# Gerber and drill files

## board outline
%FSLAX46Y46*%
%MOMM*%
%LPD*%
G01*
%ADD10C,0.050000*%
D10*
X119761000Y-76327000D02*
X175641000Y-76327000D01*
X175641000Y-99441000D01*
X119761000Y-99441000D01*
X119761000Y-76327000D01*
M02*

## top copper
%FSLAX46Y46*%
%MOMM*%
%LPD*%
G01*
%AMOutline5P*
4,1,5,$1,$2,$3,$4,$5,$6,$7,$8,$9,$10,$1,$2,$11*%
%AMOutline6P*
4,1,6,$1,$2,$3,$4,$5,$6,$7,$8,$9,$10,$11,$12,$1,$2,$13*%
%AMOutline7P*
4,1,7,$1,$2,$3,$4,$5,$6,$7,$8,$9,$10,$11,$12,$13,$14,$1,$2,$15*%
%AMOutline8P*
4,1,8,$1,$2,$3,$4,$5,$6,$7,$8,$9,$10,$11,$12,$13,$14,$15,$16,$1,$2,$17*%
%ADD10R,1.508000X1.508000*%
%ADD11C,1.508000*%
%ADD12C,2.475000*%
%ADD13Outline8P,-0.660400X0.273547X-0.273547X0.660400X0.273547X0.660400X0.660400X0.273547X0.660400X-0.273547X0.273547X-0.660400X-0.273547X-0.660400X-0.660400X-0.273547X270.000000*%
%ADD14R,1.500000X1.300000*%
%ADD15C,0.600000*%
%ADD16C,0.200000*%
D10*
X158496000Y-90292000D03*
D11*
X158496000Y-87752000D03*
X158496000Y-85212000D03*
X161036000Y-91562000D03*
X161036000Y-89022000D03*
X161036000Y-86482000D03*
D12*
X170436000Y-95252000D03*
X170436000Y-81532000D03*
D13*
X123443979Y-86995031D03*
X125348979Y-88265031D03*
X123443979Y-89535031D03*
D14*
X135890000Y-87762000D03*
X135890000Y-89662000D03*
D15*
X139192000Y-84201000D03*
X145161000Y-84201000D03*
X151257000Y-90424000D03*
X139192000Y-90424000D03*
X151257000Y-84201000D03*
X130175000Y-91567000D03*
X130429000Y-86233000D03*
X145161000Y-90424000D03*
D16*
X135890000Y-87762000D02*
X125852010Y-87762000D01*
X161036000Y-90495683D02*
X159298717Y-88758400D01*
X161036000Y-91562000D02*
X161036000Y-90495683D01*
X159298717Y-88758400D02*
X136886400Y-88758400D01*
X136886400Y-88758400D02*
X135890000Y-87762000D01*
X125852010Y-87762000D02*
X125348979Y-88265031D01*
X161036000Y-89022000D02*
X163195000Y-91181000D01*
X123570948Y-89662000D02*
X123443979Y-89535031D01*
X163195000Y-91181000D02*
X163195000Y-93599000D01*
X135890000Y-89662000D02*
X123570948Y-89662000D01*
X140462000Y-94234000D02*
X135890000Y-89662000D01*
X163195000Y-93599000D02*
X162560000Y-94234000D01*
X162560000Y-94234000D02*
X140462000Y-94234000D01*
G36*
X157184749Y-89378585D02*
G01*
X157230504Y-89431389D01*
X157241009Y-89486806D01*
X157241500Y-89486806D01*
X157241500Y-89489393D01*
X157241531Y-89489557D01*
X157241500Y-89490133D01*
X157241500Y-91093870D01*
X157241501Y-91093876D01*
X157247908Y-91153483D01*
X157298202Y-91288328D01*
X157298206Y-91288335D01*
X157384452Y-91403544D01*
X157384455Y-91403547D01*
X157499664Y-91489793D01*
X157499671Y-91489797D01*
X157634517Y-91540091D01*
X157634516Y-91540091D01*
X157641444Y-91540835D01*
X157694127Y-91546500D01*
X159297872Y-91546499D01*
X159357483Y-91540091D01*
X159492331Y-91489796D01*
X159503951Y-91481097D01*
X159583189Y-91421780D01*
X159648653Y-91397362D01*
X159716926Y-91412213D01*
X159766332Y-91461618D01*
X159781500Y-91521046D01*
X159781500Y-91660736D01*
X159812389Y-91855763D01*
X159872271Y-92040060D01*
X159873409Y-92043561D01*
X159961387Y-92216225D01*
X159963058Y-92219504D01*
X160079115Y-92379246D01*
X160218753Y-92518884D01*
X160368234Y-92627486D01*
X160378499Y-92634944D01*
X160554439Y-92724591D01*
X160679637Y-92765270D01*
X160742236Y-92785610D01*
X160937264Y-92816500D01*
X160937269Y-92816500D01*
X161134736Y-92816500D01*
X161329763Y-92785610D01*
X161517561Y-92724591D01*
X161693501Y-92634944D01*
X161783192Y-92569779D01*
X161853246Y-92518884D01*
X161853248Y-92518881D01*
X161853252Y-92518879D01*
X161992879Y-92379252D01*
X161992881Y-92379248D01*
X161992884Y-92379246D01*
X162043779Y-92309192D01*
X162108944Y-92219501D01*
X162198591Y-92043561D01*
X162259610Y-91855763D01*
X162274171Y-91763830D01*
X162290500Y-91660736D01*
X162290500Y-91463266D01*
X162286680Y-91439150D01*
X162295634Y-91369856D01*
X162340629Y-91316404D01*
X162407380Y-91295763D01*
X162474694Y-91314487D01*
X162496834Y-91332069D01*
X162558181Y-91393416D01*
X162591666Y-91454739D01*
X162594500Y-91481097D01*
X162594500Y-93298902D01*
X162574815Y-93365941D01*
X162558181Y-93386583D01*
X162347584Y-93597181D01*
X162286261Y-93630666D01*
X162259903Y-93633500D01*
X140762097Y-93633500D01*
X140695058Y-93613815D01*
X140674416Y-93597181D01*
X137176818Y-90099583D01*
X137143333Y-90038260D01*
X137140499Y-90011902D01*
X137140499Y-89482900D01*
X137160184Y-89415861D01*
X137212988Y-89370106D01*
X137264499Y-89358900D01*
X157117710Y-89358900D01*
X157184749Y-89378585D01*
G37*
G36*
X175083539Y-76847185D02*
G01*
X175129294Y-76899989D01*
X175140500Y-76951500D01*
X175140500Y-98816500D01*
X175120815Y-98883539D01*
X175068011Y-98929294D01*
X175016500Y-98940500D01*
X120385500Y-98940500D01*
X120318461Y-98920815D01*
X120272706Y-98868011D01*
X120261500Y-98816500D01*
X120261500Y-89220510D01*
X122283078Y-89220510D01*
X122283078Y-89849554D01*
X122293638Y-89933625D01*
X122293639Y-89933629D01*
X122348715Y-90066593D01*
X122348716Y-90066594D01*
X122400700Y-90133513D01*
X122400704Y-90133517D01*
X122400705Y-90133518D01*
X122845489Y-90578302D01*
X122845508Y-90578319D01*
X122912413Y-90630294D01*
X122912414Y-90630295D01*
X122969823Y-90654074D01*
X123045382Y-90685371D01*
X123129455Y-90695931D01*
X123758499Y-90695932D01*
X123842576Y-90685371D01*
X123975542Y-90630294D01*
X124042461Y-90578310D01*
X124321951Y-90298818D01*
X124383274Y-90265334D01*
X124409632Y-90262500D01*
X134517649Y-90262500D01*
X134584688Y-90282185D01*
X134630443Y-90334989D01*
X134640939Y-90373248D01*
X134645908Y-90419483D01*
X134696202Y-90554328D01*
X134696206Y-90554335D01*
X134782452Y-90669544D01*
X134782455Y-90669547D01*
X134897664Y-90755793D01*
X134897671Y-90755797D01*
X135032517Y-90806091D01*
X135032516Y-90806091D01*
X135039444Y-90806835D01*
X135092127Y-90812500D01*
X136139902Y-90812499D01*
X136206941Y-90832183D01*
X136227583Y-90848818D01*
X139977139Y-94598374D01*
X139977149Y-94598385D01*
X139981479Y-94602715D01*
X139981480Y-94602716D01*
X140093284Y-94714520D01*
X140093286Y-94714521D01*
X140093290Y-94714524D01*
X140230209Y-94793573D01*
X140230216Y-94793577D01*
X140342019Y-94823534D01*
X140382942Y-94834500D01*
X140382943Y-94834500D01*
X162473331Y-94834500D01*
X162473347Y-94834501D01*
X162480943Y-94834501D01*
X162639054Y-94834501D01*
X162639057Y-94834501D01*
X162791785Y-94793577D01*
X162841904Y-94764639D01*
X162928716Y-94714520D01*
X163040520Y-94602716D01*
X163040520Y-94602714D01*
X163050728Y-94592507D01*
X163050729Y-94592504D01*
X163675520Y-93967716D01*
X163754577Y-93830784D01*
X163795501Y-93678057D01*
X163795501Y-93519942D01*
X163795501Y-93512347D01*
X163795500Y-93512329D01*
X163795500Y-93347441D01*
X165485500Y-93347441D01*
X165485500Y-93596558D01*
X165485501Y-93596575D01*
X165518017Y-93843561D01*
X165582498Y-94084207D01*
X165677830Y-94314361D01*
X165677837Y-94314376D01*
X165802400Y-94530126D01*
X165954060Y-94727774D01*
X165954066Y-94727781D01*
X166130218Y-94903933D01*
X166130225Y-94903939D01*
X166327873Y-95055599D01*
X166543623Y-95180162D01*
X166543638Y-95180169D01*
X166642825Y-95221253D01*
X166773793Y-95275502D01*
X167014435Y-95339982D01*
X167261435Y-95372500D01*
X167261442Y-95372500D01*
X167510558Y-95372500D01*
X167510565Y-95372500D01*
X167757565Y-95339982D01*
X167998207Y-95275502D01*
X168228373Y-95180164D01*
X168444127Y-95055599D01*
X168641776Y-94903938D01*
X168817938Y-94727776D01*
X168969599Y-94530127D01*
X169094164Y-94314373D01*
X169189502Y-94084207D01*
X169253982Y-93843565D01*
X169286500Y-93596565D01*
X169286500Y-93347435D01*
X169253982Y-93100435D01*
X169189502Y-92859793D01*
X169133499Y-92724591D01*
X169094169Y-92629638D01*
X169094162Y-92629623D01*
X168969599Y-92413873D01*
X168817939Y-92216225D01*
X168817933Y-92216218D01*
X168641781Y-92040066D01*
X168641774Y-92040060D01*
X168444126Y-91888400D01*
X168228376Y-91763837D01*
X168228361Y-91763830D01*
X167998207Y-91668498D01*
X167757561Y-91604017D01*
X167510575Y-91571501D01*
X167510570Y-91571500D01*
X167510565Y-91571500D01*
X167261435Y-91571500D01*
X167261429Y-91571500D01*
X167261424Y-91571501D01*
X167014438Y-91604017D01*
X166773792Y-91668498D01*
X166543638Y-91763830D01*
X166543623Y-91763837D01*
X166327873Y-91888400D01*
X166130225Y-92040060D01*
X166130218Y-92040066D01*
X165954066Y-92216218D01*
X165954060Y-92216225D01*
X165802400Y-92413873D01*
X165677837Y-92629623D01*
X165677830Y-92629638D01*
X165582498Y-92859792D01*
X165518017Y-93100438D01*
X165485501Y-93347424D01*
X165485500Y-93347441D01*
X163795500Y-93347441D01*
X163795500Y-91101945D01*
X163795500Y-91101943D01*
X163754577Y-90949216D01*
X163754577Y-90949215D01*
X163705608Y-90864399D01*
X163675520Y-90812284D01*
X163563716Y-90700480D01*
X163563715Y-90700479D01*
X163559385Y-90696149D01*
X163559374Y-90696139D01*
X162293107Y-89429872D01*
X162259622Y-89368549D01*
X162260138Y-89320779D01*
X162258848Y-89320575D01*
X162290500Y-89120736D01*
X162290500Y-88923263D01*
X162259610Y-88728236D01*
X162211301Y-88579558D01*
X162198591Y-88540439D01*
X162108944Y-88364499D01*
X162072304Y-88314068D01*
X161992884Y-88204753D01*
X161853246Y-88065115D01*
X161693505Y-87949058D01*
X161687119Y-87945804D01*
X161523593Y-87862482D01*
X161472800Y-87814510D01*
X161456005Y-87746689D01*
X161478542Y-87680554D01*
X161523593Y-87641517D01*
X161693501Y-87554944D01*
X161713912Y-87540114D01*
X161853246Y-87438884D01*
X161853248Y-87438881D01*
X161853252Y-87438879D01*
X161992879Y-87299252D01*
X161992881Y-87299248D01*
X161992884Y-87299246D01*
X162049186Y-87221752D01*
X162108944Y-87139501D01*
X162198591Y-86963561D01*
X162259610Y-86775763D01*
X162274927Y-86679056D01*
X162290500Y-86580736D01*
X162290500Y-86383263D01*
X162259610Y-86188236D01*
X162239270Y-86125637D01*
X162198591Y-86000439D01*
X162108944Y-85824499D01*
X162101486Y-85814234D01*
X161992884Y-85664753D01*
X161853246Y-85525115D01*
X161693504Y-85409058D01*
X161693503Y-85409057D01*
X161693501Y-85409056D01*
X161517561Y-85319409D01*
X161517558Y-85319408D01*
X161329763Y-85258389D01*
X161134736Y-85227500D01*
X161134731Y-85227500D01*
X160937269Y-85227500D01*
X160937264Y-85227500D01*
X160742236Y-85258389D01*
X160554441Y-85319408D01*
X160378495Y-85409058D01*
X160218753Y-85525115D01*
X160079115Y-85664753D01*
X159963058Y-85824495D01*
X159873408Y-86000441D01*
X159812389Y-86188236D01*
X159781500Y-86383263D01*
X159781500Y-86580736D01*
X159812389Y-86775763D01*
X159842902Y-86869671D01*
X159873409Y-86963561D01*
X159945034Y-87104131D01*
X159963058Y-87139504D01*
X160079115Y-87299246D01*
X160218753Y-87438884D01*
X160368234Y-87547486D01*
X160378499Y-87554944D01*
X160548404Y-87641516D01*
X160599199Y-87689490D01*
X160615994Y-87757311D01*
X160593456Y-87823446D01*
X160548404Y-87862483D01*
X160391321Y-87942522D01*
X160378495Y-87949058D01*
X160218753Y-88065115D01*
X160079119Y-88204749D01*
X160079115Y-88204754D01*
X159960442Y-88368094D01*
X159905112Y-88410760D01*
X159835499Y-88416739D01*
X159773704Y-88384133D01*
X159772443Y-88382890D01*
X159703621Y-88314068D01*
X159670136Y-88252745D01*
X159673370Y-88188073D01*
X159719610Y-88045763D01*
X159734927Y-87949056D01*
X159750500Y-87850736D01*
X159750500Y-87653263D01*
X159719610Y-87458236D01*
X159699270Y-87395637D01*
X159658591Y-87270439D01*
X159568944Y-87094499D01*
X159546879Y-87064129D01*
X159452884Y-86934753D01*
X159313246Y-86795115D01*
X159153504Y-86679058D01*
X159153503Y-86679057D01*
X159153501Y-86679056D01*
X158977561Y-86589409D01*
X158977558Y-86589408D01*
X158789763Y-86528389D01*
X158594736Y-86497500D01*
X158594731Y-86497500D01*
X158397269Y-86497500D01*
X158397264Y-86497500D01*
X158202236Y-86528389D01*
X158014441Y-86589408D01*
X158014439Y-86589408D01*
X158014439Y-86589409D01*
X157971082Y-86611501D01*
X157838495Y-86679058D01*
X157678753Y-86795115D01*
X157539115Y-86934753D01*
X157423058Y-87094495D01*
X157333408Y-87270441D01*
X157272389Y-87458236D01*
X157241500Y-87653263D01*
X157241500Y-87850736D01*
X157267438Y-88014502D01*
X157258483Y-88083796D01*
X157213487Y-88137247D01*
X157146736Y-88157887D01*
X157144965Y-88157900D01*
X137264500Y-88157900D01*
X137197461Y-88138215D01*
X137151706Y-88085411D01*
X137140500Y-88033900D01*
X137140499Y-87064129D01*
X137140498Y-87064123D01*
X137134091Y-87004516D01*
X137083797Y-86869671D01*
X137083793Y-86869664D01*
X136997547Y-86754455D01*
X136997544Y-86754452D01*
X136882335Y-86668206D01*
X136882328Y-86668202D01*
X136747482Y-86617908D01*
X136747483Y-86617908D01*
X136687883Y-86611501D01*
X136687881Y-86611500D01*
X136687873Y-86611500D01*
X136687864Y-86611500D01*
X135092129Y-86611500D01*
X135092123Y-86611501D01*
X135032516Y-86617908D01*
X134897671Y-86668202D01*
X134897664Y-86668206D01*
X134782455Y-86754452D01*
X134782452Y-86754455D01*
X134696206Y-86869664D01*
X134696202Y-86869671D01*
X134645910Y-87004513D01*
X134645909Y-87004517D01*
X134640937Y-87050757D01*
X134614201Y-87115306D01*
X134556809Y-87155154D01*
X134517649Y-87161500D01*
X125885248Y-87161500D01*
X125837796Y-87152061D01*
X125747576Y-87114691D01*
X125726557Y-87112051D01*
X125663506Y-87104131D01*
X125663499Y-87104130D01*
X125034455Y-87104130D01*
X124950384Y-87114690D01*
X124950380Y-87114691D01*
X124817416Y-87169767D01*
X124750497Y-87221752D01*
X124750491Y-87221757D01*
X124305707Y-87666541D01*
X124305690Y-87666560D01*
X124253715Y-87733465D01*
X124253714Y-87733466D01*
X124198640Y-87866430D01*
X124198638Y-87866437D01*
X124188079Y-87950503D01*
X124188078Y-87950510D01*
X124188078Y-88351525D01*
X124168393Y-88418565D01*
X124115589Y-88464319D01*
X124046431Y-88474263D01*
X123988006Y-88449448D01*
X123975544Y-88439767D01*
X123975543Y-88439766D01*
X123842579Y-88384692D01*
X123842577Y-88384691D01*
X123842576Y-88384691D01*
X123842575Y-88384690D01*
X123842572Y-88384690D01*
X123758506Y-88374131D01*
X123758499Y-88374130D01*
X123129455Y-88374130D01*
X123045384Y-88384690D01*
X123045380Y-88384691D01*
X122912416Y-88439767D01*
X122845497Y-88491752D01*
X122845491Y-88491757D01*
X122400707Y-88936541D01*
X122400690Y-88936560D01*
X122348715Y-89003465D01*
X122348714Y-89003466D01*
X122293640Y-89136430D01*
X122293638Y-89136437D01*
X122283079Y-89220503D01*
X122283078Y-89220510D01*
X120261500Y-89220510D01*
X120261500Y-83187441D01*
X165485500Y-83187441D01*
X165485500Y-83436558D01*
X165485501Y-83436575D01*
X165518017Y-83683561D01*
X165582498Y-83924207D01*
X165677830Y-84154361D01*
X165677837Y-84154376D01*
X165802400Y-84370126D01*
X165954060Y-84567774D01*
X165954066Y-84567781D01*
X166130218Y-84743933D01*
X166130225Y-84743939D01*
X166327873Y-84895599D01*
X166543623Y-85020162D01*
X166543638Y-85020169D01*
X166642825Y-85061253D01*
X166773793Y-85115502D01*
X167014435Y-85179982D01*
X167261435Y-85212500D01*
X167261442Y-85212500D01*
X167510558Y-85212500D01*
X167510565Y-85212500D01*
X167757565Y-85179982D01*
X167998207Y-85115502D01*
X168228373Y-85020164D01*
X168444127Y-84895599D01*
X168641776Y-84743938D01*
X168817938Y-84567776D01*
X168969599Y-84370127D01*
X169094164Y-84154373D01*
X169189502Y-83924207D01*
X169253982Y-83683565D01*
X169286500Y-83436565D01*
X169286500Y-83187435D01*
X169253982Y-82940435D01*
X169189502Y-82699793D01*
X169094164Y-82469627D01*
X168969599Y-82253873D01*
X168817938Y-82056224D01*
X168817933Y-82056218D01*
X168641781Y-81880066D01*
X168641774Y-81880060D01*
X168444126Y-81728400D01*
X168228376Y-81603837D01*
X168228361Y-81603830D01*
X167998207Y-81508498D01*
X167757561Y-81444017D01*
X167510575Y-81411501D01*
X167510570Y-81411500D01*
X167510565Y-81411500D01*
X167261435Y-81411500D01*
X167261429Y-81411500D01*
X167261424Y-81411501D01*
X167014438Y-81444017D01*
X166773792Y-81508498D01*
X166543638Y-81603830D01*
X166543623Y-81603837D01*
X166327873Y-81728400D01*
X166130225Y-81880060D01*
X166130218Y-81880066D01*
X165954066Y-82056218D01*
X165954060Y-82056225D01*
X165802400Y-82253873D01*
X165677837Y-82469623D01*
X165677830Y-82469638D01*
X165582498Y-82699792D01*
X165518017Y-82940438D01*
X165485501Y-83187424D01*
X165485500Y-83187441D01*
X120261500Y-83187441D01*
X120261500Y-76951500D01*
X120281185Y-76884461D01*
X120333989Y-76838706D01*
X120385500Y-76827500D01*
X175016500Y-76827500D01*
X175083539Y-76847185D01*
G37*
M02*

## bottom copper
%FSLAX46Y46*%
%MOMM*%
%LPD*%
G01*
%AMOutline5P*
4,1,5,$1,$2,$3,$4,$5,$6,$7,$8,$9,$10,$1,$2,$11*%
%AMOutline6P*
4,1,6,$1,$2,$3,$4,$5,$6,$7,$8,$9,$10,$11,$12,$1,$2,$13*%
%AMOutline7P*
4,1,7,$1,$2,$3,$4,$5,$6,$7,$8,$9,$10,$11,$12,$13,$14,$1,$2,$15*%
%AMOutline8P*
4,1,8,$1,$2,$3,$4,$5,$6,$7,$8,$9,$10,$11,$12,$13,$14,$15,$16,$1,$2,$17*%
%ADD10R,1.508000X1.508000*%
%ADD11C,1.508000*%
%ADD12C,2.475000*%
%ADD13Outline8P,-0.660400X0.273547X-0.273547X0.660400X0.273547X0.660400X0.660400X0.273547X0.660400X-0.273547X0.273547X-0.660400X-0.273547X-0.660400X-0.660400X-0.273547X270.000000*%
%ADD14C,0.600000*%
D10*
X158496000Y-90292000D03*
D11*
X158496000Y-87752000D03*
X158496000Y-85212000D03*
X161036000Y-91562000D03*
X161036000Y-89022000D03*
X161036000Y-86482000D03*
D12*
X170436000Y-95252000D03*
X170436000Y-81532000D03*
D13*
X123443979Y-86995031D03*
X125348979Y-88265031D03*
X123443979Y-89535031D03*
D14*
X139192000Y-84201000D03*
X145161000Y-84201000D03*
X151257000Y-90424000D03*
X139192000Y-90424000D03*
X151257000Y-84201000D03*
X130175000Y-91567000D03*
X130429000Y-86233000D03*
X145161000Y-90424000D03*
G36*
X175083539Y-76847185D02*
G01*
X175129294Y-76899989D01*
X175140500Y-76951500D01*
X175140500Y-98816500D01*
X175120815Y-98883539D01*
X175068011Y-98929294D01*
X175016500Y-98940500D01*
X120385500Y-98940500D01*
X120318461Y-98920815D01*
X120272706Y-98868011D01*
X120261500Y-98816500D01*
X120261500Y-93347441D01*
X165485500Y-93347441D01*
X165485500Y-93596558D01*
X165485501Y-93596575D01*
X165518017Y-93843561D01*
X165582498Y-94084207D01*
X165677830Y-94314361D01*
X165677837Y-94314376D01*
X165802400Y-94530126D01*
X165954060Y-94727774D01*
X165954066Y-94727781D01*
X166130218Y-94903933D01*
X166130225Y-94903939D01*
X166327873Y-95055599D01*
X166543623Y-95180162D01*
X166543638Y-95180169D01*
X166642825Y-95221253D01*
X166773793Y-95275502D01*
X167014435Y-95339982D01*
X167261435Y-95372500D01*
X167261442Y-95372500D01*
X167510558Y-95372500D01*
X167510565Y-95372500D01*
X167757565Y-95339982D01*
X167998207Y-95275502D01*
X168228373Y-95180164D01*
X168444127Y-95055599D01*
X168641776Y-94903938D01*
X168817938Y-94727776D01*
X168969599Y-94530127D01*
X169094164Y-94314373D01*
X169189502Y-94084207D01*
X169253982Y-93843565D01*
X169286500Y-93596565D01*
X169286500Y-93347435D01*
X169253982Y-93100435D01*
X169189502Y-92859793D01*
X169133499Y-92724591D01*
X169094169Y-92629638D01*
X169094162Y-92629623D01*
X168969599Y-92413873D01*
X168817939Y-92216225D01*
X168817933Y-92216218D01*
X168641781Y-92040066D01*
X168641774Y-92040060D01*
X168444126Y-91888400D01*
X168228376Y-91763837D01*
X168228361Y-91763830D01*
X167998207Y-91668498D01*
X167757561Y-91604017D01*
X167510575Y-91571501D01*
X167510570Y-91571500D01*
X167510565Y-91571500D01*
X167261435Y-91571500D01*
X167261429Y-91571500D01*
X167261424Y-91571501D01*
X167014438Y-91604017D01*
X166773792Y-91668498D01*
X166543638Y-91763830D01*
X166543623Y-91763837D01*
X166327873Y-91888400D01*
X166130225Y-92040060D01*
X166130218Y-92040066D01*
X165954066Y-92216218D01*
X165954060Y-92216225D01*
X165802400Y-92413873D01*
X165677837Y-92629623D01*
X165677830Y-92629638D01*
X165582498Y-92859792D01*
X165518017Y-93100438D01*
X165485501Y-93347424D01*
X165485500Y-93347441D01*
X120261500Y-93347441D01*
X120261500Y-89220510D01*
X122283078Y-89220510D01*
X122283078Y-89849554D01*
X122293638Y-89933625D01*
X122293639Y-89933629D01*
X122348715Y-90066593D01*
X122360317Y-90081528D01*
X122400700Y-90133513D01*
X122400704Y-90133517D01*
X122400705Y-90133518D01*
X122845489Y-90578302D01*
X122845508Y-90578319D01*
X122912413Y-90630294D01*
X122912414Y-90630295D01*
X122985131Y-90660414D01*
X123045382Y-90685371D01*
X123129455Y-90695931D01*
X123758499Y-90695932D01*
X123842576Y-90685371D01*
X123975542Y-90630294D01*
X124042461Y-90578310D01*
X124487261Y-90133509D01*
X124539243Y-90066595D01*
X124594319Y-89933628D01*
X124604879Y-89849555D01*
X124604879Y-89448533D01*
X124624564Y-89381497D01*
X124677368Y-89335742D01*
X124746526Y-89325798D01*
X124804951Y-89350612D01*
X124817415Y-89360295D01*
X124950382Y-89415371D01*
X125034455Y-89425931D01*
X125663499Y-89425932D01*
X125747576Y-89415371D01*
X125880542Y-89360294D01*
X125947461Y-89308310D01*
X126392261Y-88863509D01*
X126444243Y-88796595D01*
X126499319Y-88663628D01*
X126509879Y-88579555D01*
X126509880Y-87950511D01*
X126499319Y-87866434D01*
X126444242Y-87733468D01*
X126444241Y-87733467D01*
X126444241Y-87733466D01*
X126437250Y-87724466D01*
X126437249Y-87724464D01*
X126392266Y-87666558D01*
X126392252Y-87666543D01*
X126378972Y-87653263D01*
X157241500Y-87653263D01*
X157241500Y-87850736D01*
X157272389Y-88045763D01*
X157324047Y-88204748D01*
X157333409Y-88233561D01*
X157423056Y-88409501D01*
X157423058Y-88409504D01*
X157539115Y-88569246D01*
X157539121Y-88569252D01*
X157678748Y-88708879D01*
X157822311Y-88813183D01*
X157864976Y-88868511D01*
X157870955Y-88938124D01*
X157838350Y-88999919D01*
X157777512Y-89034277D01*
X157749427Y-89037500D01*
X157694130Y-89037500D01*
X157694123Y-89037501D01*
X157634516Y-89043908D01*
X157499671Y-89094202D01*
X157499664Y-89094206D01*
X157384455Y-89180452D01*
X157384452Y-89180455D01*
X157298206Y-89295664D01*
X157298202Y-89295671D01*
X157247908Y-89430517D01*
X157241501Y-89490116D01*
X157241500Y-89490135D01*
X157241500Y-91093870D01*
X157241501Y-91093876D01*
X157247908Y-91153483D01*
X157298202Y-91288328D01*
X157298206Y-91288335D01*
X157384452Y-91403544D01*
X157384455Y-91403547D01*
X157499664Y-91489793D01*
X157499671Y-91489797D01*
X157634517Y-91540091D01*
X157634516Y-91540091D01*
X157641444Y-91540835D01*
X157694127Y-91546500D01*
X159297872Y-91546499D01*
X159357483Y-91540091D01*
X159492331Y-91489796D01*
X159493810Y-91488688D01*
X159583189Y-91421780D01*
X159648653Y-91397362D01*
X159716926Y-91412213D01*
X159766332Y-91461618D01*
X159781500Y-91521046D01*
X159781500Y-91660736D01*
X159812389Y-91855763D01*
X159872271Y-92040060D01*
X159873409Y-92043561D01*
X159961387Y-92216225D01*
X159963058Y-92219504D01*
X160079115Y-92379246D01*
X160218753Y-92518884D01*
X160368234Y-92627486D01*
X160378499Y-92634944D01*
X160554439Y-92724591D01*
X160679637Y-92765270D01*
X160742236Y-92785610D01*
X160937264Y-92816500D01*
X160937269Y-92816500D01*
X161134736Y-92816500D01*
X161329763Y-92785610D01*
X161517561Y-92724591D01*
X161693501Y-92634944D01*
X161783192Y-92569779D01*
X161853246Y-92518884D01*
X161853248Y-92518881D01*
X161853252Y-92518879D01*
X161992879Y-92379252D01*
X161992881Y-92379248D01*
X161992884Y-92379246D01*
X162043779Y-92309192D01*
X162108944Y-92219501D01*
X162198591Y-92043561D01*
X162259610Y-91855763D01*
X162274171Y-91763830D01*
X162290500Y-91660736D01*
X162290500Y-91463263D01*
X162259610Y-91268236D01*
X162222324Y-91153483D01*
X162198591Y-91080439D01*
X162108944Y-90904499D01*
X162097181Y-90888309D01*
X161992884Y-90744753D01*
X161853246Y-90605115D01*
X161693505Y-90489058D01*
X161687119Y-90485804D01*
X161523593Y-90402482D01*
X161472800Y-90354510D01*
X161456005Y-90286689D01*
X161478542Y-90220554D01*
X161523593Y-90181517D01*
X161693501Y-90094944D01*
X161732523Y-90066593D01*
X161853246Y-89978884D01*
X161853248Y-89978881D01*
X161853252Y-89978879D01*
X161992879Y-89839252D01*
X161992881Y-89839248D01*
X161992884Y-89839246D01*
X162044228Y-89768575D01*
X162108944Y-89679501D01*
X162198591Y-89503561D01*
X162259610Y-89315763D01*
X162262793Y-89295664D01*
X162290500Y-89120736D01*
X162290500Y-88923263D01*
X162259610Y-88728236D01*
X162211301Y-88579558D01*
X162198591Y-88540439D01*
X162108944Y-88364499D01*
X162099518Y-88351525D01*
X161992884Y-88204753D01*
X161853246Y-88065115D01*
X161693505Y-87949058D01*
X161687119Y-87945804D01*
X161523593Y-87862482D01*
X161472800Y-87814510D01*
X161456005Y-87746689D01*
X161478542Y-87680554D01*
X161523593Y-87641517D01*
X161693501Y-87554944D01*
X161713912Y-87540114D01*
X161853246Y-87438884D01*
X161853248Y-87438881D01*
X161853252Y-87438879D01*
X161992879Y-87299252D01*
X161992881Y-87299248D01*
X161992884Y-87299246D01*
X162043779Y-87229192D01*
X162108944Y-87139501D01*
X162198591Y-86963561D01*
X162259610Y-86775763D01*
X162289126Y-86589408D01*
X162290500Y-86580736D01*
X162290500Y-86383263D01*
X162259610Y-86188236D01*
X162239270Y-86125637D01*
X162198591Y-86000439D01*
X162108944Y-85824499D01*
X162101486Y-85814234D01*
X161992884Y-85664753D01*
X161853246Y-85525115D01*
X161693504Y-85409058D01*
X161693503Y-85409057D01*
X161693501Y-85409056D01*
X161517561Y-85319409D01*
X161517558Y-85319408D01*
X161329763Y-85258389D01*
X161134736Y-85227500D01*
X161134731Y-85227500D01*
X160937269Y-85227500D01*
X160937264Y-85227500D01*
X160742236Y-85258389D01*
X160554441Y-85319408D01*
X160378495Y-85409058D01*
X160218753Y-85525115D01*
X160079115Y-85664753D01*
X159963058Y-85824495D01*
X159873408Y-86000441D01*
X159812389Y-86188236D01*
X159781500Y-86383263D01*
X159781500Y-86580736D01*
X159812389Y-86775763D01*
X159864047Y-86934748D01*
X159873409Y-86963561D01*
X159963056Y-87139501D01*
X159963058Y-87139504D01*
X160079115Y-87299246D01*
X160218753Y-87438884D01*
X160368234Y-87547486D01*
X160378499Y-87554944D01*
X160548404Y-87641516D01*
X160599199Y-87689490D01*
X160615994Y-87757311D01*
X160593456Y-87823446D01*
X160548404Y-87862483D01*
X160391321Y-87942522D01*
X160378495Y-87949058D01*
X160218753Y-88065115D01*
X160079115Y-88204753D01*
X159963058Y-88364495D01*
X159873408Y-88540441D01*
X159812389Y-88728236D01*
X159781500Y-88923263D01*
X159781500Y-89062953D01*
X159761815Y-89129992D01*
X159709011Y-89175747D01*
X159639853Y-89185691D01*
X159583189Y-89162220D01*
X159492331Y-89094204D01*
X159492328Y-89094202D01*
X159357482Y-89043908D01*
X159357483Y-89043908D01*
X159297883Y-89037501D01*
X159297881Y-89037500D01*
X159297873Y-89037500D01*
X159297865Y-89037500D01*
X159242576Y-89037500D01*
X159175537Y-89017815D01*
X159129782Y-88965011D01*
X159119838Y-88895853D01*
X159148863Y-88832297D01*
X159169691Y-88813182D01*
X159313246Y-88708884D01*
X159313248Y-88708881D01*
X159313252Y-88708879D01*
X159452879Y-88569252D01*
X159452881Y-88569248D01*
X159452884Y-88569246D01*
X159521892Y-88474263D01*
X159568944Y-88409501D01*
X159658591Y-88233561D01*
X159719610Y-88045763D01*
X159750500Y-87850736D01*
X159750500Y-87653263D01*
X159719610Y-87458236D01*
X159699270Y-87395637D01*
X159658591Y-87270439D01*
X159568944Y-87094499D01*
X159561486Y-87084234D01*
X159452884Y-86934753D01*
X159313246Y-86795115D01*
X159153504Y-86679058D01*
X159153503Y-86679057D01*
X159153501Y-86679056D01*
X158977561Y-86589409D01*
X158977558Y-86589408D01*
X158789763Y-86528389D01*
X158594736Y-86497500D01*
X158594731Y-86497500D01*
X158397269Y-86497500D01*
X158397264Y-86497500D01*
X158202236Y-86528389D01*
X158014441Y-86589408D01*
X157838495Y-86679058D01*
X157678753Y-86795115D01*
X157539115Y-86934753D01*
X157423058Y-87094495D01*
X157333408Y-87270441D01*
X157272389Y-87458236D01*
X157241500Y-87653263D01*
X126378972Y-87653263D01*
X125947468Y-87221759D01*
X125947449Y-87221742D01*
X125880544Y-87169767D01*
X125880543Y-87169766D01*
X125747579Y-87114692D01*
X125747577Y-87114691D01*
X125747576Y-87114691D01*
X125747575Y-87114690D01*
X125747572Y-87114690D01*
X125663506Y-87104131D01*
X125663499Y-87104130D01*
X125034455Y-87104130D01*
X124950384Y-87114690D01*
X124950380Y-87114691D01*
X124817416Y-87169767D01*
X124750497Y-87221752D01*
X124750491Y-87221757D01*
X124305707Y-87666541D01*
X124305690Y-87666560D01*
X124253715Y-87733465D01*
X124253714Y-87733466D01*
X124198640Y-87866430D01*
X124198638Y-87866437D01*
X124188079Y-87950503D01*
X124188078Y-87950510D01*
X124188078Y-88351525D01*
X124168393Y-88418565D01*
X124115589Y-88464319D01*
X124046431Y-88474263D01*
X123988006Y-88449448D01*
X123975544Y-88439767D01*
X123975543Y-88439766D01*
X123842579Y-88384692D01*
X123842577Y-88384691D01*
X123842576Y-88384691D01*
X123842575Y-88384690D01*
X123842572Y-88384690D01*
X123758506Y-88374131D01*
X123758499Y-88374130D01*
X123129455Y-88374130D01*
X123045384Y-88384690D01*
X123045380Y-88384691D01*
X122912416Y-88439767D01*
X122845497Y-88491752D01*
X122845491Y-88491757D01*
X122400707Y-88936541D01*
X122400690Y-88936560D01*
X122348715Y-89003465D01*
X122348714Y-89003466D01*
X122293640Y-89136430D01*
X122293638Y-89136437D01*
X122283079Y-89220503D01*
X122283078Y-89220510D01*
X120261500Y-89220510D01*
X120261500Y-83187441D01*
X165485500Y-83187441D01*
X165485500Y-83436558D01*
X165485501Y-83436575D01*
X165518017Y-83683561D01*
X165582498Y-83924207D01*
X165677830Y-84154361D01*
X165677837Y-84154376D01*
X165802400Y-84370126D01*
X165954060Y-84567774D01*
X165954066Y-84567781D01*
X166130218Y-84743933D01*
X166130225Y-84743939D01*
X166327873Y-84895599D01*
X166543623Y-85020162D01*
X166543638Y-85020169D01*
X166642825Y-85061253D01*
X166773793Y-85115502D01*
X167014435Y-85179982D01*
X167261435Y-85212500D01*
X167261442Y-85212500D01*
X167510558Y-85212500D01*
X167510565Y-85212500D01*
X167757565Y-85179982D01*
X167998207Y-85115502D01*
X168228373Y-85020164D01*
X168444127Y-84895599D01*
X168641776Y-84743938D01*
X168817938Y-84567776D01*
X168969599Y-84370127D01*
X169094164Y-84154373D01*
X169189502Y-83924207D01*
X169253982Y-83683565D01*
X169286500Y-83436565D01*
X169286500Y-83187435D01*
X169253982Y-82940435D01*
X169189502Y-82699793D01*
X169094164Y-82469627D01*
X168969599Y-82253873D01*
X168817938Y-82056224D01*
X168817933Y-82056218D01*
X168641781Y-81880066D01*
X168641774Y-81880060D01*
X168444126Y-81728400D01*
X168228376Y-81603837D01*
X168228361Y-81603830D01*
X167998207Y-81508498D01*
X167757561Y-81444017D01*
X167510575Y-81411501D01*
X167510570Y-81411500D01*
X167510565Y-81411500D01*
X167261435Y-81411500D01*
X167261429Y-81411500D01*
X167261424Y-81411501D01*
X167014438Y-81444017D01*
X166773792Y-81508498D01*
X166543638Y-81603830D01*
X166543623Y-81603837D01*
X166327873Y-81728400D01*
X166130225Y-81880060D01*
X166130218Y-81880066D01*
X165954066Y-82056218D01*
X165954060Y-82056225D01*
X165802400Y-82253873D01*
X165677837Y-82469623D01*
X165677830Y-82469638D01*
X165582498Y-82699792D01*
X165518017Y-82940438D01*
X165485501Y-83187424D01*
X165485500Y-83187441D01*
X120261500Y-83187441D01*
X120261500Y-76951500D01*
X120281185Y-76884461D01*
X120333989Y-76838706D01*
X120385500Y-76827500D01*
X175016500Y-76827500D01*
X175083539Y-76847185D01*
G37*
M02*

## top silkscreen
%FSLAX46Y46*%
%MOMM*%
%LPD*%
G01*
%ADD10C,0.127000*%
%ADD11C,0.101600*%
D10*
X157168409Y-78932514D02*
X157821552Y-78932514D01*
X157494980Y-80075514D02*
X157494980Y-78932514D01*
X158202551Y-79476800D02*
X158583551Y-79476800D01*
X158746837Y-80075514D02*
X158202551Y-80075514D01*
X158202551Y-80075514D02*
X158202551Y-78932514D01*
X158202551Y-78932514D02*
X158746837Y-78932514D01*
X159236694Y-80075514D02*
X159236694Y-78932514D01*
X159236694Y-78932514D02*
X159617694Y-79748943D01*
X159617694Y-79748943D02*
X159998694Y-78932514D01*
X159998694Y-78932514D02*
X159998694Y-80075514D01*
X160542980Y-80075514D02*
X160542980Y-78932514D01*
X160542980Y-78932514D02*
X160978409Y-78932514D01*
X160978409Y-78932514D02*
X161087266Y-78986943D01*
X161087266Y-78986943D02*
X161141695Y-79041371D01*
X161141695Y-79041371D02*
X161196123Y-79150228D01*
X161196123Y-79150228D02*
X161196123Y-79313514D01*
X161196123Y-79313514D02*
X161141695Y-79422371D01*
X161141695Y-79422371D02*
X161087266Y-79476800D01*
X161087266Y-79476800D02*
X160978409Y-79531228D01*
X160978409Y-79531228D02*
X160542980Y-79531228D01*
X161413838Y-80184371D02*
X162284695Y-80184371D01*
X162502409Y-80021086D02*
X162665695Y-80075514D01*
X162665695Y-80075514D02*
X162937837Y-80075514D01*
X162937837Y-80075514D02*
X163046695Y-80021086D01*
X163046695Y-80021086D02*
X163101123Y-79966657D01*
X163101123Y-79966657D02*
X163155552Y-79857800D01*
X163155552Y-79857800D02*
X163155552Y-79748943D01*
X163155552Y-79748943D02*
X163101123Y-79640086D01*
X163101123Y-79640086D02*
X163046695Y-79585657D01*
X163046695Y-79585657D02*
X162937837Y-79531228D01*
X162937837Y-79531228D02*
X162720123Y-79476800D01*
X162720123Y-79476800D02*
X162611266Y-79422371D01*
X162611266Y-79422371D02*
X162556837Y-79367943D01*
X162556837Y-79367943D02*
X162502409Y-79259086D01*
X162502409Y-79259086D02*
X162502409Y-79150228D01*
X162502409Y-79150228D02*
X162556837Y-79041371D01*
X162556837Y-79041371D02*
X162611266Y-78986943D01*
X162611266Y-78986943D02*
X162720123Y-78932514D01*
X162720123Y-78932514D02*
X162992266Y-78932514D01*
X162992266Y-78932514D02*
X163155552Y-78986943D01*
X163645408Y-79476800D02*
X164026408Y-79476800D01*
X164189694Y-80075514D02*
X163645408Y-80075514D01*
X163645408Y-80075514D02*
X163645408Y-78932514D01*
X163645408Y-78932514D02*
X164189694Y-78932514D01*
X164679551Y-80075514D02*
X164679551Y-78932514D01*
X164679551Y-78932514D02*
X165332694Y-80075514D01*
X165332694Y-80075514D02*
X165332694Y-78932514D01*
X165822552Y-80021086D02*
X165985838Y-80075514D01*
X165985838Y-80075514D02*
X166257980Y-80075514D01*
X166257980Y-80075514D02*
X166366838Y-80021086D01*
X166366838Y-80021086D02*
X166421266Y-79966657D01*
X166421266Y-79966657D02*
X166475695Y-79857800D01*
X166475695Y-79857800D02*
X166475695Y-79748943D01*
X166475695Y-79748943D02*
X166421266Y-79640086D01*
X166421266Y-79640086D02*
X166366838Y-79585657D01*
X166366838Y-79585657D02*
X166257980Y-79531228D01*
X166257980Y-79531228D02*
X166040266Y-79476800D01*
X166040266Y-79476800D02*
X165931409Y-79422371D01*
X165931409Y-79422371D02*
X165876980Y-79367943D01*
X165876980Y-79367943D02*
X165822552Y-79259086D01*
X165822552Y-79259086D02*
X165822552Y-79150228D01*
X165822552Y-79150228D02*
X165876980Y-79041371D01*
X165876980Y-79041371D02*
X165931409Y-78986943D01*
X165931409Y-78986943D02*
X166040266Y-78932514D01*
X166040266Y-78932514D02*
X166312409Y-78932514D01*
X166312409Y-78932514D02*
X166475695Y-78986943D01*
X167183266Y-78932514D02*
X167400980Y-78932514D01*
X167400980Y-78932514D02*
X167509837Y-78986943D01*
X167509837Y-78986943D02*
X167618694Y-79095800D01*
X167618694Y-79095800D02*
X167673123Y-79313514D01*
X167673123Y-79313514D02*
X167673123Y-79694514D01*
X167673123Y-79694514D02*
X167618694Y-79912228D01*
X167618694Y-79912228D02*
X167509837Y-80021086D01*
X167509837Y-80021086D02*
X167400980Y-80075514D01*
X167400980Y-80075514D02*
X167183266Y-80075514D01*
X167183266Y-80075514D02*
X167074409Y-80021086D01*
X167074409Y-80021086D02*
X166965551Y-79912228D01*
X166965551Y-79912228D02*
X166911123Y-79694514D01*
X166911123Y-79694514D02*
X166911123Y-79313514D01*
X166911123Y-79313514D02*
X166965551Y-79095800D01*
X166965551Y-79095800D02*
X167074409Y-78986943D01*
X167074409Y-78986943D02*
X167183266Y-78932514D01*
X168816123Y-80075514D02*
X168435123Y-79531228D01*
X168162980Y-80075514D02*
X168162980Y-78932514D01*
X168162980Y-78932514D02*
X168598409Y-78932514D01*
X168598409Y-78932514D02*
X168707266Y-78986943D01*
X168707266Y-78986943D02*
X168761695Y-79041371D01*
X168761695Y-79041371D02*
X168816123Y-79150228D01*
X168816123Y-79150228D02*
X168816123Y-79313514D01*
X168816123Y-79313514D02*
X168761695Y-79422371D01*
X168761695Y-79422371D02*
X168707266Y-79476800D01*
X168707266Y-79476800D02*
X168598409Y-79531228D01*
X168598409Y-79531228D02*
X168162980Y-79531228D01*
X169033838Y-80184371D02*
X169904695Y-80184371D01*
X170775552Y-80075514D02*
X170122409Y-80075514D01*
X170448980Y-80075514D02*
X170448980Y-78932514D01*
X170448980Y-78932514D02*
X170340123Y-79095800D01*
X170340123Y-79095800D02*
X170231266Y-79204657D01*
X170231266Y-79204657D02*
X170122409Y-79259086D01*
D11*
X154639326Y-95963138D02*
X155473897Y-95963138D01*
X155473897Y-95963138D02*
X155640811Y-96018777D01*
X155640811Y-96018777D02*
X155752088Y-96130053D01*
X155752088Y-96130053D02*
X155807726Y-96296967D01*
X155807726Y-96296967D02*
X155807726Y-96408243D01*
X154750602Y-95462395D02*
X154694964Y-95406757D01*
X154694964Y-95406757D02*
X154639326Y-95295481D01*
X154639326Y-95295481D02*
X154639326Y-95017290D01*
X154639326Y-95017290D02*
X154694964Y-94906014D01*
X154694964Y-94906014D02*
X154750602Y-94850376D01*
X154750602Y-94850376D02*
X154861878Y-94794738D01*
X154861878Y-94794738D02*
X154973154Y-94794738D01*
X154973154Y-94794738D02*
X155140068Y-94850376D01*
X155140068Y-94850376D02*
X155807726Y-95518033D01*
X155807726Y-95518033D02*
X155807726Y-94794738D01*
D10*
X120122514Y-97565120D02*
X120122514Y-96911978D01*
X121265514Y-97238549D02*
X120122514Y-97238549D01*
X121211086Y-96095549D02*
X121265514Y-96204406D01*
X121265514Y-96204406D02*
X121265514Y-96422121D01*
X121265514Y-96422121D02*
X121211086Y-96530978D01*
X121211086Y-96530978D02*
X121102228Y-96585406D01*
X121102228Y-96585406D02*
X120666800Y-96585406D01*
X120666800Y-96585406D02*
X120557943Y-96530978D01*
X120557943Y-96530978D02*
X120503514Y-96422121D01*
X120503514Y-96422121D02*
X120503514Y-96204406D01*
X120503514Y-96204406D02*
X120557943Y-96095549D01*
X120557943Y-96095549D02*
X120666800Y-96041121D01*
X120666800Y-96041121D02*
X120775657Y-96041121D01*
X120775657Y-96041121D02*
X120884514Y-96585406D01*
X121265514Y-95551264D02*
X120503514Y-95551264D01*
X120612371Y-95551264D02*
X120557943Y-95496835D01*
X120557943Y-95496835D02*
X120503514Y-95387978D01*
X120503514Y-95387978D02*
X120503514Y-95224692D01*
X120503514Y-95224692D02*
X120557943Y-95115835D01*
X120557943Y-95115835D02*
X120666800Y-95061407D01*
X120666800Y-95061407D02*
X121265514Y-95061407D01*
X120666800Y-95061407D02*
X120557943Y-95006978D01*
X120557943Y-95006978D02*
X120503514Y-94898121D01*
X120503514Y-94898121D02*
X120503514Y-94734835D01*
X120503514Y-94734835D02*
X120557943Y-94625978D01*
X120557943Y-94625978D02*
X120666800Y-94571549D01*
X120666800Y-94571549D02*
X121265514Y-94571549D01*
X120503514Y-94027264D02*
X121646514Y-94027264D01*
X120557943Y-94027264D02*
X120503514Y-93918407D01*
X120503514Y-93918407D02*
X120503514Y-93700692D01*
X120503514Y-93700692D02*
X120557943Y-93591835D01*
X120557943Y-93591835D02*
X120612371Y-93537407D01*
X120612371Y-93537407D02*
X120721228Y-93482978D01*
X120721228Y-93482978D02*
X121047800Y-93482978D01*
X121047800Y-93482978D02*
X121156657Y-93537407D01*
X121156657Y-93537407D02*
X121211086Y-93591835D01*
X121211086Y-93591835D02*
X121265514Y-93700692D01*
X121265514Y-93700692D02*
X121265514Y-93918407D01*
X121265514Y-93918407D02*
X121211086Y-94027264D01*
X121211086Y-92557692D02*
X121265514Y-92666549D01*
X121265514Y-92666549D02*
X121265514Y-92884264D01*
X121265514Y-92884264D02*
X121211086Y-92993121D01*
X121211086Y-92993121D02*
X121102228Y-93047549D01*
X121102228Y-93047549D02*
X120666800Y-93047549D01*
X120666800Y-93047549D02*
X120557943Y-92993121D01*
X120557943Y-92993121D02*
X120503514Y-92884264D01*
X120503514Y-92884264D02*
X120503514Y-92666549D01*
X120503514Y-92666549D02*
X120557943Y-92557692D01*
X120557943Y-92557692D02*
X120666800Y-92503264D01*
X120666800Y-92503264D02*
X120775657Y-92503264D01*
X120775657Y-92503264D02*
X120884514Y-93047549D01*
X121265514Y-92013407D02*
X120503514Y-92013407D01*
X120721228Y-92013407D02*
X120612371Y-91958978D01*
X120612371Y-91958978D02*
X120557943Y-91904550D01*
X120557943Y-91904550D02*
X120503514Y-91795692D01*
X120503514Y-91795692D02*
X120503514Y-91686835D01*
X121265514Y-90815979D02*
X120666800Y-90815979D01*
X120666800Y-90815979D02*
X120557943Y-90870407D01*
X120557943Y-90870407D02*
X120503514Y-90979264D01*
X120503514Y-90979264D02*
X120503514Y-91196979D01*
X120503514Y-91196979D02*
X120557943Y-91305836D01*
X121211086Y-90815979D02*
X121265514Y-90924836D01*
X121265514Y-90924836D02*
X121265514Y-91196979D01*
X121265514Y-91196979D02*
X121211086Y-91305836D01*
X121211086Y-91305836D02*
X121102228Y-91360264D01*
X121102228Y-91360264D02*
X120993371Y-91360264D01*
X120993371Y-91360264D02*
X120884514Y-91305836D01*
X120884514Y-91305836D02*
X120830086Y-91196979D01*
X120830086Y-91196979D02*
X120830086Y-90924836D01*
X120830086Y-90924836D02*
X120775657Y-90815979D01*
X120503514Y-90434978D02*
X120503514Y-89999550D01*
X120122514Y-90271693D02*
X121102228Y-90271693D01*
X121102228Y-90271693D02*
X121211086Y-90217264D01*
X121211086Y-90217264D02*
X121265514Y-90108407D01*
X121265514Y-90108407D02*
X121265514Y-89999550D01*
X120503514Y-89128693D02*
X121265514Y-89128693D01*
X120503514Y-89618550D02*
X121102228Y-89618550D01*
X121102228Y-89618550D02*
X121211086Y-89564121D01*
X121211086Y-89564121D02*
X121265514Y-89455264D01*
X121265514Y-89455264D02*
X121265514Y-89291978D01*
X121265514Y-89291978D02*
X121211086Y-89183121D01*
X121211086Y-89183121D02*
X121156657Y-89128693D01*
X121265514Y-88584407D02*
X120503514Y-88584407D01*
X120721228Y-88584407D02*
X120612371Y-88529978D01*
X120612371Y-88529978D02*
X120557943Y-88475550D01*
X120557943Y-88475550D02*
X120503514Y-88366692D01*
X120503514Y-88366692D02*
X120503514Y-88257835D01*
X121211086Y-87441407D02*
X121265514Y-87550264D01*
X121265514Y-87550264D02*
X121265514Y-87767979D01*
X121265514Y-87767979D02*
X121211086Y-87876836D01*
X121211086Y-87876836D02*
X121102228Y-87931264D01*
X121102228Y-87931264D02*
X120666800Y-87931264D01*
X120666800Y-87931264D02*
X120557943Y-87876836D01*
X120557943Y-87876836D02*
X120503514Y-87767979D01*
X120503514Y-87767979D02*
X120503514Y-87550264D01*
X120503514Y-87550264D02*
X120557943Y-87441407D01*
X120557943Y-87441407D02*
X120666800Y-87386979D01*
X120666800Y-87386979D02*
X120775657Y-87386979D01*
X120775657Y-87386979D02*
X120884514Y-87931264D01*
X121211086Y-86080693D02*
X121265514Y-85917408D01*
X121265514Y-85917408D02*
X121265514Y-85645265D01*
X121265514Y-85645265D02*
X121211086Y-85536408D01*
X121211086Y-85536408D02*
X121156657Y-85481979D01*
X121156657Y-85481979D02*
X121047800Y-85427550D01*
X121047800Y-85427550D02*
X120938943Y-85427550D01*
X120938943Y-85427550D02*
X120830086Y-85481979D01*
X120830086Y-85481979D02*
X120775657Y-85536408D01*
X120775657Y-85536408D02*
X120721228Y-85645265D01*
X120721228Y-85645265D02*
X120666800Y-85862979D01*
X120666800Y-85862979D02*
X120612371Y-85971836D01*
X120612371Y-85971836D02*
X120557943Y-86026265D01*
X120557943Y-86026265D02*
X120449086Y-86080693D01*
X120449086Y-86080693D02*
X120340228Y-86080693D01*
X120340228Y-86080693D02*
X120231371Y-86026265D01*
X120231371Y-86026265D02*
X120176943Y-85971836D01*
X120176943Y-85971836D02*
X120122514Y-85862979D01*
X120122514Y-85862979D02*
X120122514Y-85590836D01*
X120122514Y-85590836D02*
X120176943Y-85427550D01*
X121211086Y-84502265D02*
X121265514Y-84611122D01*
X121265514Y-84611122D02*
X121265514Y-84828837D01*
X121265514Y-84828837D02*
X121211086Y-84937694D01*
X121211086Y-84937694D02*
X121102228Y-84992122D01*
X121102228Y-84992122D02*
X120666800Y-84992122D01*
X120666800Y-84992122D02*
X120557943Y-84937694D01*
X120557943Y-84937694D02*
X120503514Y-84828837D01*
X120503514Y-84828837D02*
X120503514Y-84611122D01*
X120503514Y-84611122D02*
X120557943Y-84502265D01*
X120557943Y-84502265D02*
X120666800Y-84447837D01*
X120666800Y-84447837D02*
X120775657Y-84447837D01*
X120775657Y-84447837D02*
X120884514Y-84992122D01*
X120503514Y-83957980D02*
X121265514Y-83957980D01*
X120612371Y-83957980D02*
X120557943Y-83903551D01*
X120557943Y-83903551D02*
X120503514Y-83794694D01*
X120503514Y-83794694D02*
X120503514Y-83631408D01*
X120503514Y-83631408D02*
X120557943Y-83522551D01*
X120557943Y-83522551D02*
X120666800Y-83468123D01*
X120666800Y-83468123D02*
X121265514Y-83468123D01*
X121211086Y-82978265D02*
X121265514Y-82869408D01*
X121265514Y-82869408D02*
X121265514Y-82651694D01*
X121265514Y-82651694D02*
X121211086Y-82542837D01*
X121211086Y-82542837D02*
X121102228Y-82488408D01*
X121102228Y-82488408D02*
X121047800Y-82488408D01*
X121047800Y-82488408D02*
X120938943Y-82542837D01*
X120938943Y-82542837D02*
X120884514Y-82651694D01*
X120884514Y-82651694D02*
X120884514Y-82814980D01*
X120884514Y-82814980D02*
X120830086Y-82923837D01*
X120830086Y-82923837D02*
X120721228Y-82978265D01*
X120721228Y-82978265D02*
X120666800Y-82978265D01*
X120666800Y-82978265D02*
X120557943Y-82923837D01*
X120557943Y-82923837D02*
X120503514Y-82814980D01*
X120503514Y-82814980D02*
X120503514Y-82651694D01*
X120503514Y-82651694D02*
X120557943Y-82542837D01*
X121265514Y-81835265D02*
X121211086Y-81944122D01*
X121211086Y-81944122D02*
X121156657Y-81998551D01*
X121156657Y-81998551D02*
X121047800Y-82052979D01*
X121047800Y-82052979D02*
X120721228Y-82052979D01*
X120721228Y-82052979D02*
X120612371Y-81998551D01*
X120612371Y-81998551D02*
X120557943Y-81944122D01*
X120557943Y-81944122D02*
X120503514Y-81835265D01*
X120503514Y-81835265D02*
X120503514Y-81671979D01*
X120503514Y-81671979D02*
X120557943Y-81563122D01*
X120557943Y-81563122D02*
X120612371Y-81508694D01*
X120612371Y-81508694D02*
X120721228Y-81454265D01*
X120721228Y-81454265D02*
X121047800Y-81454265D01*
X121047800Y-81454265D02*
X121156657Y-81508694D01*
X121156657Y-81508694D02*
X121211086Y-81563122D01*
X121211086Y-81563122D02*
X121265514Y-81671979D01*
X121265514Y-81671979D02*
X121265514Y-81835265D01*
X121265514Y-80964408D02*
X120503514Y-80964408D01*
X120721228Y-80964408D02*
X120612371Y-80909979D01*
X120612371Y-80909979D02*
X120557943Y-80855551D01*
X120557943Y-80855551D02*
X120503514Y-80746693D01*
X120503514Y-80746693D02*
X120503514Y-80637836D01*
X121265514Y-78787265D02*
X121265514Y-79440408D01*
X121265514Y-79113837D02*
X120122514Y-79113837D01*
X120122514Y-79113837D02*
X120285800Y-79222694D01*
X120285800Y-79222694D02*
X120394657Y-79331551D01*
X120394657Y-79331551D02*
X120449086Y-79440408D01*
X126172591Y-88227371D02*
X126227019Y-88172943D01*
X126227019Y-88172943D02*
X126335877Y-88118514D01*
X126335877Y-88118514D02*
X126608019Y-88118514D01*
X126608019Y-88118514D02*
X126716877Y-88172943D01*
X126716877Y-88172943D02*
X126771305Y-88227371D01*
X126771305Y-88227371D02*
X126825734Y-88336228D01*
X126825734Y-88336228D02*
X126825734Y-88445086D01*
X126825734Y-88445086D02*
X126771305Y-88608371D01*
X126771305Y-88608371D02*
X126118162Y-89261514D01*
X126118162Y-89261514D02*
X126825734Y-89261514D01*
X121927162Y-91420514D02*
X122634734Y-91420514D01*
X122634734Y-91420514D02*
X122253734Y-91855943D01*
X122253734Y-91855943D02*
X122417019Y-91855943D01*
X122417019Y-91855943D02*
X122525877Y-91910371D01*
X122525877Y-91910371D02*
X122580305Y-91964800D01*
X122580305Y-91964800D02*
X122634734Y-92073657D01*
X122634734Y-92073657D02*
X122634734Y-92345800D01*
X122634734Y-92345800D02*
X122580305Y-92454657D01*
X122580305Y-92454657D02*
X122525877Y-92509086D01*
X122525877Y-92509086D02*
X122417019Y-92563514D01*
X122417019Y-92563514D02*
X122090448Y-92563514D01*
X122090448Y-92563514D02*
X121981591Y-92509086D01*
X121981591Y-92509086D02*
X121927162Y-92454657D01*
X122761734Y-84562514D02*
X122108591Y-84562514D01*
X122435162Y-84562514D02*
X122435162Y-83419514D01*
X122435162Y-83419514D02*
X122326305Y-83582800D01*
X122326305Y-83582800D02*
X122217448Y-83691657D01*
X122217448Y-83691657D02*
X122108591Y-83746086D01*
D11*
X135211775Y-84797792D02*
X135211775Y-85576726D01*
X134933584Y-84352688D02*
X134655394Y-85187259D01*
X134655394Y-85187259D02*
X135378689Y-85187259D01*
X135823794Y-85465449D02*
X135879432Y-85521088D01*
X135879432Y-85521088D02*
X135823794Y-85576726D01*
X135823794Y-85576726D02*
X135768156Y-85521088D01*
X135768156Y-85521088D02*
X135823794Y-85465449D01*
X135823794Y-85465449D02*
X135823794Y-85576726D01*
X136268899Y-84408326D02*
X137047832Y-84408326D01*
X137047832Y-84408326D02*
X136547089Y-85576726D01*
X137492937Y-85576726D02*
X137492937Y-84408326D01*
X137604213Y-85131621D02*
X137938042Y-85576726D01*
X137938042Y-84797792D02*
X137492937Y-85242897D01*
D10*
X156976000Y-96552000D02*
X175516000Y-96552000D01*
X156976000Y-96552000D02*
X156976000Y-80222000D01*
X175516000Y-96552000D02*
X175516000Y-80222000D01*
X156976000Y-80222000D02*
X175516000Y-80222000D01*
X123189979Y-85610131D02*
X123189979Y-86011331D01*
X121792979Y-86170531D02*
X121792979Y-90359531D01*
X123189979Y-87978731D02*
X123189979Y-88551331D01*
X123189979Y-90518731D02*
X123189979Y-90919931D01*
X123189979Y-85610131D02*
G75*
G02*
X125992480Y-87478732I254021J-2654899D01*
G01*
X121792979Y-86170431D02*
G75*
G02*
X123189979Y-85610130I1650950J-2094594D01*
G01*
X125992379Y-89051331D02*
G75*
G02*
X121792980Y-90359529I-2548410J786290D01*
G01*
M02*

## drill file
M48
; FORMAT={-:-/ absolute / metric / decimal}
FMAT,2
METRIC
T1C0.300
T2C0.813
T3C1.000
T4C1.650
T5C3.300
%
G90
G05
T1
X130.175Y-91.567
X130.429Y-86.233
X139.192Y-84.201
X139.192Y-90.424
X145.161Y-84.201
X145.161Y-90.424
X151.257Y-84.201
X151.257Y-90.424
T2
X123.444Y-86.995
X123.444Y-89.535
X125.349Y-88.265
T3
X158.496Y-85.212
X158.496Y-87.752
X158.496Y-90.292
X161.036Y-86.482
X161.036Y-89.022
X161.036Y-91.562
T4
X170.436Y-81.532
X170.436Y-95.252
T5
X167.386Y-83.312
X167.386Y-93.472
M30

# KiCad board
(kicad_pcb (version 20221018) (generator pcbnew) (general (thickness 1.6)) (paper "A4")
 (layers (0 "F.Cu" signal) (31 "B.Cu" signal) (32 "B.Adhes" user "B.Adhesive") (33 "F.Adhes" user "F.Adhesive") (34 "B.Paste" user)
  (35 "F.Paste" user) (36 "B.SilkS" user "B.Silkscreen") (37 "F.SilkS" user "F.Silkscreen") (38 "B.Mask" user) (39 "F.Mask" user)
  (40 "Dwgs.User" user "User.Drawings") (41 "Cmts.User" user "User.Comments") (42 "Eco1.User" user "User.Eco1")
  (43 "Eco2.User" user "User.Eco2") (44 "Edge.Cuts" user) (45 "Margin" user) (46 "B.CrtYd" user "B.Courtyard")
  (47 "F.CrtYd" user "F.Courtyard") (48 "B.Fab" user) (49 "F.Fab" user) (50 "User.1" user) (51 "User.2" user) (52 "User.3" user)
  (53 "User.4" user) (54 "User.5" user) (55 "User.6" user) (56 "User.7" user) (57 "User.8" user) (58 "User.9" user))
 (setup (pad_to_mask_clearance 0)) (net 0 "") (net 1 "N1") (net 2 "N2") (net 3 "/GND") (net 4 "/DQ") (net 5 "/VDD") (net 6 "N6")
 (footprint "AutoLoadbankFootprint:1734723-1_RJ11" (layer "F.Cu") (at 161.036 87.752 90)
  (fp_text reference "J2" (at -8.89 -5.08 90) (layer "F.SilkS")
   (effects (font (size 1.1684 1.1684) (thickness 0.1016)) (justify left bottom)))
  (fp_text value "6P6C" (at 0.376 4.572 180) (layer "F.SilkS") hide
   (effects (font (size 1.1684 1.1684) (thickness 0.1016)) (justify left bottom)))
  (fp_line (start -8.8 -4.06) (end -8.8 14.48) (stroke (width 0.127) (type solid)) (layer "F.SilkS"))
  (fp_line (start -8.8 -4.06) (end 7.53 -4.06) (stroke (width 0.127) (type solid)) (layer "F.SilkS"))
  (fp_line (start -8.8 14.48) (end 7.53 14.48) (stroke (width 0.127) (type solid)) (layer "F.SilkS"))
  (fp_line (start 7.53 -4.06) (end 7.53 14.48) (stroke (width 0.127) (type solid)) (layer "F.SilkS"))
  (pad "" np_thru_hole circle (at -5.72 6.35 90) (size 3.3 3.3) (drill 3.3) (layers "*.Cu" "*.Mask"))
  (pad "" np_thru_hole circle (at 4.44 6.35 90) (size 3.3 3.3) (drill 3.3) (layers "*.Cu" "*.Mask"))
  (pad "1" thru_hole rect (at -2.54 -2.54 90) (size 1.508 1.508) (drill 1) (layers "*.Cu" "*.Mask") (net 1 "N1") (solder_mask_margin 0.1016)
   (thermal_bridge_angle 45))
  (pad "2" thru_hole circle (at 0 -2.54 90) (size 1.508 1.508) (drill 1) (layers "*.Cu" "*.Mask") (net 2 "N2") (solder_mask_margin 0.1016))
  (pad "3" thru_hole circle (at 2.54 -2.54 90) (size 1.508 1.508) (drill 1) (layers "*.Cu" "*.Mask") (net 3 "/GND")
   (solder_mask_margin 0.1016))
  (pad "4" thru_hole circle (at -3.81 0 90) (size 1.508 1.508) (drill 1) (layers "*.Cu" "*.Mask") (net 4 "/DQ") (solder_mask_margin 0.1016))
  (pad "5" thru_hole circle (at -1.27 0 90) (size 1.508 1.508) (drill 1) (layers "*.Cu" "*.Mask") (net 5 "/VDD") (solder_mask_margin 0.1016))
  (pad "6" thru_hole circle (at 1.27 0 90) (size 1.508 1.508) (drill 1) (layers "*.Cu" "*.Mask") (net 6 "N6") (solder_mask_margin 0.1016))
  (pad "SH1" thru_hole circle (at -7.5 9.4 90) (size 2.475 2.475) (drill 1.65) (layers "*.Cu" "*.Mask") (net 3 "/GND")
   (solder_mask_margin 0.1016))
  (pad "SH2" thru_hole circle (at 6.22 9.4 90) (size 2.475 2.475) (drill 1.65) (layers "*.Cu" "*.Mask") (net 3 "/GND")
   (solder_mask_margin 0.1016)))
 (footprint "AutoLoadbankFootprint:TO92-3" (layer "F.Cu") (at 123.443979 88.265031 -90)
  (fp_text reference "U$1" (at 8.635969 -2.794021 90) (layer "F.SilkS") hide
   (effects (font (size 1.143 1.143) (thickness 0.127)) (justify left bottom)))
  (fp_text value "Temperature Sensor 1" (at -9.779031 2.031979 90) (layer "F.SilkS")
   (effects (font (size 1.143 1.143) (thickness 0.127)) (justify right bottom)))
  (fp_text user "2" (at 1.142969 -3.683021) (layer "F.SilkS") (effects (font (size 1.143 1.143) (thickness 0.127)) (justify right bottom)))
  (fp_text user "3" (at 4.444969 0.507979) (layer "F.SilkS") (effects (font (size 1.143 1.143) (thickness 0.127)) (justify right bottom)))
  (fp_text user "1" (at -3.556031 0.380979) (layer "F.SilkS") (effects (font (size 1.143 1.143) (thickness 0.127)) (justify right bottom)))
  (fp_line (start -2.6549 0.254) (end -2.2537 0.254) (stroke (width 0.127) (type solid)) (layer "F.SilkS"))
  (fp_line (start -2.0945 1.651) (end 2.0945 1.651) (stroke (width 0.127) (type solid)) (layer "F.SilkS"))
  (fp_line (start -0.2863 0.254) (end 0.2863 0.254) (stroke (width 0.127) (type solid)) (layer "F.SilkS"))
  (fp_line (start 2.2537 0.254) (end 2.6549 0.254) (stroke (width 0.127) (type solid)) (layer "F.SilkS"))
  (fp_arc (start -2.6549 0.254) (mid -2.219001 -1.479566) (end -0.786299 -2.548501) (stroke (width 0.127) (type solid)) (layer "F.SilkS"))
  (fp_arc (start -2.0946 1.651) (mid -2.475347 0.992847) (end -2.654901 0.254) (stroke (width 0.127) (type solid)) (layer "F.SilkS"))
  (fp_arc (start 0.7863 -2.5484) (mid 2.546274 -0.793203) (end 2.094499 1.651) (stroke (width 0.127) (type solid)) (layer "F.SilkS"))
  (pad "1" thru_hole roundrect (at -1.27 0 270) (size 1.3208 1.3208) (drill 0.8128) (layers "*.Cu" "*.Mask") (roundrect_rratio 0.25)
   (chamfer_ratio 0.2928932188) (chamfer top_left top_right bottom_left bottom_right) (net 3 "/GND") (solder_mask_margin 0.1016)
   (thermal_bridge_angle 45))
  (pad "2" thru_hole roundrect (at 0 -1.905 270) (size 1.3208 1.3208) (drill 0.8128) (layers "*.Cu" "*.Mask") (roundrect_rratio 0.25)
   (chamfer_ratio 0.2928932188) (chamfer top_left top_right bottom_left bottom_right) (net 4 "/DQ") (solder_mask_margin 0.1016)
   (thermal_bridge_angle 45))
  (pad "3" thru_hole roundrect (at 1.27 0 270) (size 1.3208 1.3208) (drill 0.8128) (layers "*.Cu" "*.Mask") (roundrect_rratio 0.25)
   (chamfer_ratio 0.2928932188) (chamfer top_left top_right bottom_left bottom_right) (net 5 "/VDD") (solder_mask_margin 0.1016)
   (thermal_bridge_angle 45)))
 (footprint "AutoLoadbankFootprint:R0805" (layer "F.Cu") (at 135.89 88.712 -90)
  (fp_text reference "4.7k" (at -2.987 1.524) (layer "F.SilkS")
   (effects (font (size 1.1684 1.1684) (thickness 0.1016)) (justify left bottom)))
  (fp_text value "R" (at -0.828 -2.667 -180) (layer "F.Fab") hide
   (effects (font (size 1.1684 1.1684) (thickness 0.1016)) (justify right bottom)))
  (pad "1" smd rect (at -0.95 0 270) (size 1.3 1.5) (layers "F.Cu" "F.Paste" "F.Mask") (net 4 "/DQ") (solder_mask_margin 0.1016)
   (thermal_bridge_angle 45))
  (pad "2" smd rect (at 0.95 0 270) (size 1.3 1.5) (layers "F.Cu" "F.Paste" "F.Mask") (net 5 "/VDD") (solder_mask_margin 0.1016)
   (thermal_bridge_angle 45)))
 (gr_rect (start 119.761 76.327) (end 175.641 99.441) (stroke (width 0.05) (type default)) (fill none) (layer "Edge.Cuts"))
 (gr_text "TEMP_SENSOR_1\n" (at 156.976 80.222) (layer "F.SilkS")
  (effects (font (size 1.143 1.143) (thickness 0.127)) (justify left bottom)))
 (via (at 139.192 84.201) (size 0.6) (drill 0.3) (layers "F.Cu" "B.Cu") (free) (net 3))
 (via (at 145.161 84.201) (size 0.6) (drill 0.3) (layers "F.Cu" "B.Cu") (free) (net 3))
 (via (at 151.257 90.424) (size 0.6) (drill 0.3) (layers "F.Cu" "B.Cu") (free) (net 3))
 (via (at 139.192 90.424) (size 0.6) (drill 0.3) (layers "F.Cu" "B.Cu") (free) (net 3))
 (via (at 151.257 84.201) (size 0.6) (drill 0.3) (layers "F.Cu" "B.Cu") (free) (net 3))
 (via (at 130.175 91.567) (size 0.6) (drill 0.3) (layers "F.Cu" "B.Cu") (free) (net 3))
 (via (at 130.429 86.233) (size 0.6) (drill 0.3) (layers "F.Cu" "B.Cu") (free) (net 3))
 (via (at 145.161 90.424) (size 0.6) (drill 0.3) (layers "F.Cu" "B.Cu") (free) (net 3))
 (segment (start 135.89 87.762) (end 125.85201 87.762) (width 0.2) (layer "F.Cu") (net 4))
 (segment (start 161.036 90.495683) (end 159.298717 88.7584) (width 0.2) (layer "F.Cu") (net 4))
 (segment (start 161.036 91.562) (end 161.036 90.495683) (width 0.2) (layer "F.Cu") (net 4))
 (segment (start 159.298717 88.7584) (end 136.8864 88.7584) (width 0.2) (layer "F.Cu") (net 4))
 (segment (start 136.8864 88.7584) (end 135.89 87.762) (width 0.2) (layer "F.Cu") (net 4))
 (segment (start 125.85201 87.762) (end 125.348979 88.265031) (width 0.2) (layer "F.Cu") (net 4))
 (segment (start 161.036 89.022) (end 163.195 91.181) (width 0.2) (layer "F.Cu") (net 5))
 (segment (start 123.570948 89.662) (end 123.443979 89.535031) (width 0.2) (layer "F.Cu") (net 5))
 (segment (start 163.195 91.181) (end 163.195 93.599) (width 0.2) (layer "F.Cu") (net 5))
 (segment (start 135.89 89.662) (end 123.570948 89.662) (width 0.2) (layer "F.Cu") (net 5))
 (segment (start 140.462 94.234) (end 135.89 89.662) (width 0.2) (layer "F.Cu") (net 5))
 (segment (start 163.195 93.599) (end 162.56 94.234) (width 0.2) (layer "F.Cu") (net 5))
 (segment (start 162.56 94.234) (end 140.462 94.234) (width 0.2) (layer "F.Cu") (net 5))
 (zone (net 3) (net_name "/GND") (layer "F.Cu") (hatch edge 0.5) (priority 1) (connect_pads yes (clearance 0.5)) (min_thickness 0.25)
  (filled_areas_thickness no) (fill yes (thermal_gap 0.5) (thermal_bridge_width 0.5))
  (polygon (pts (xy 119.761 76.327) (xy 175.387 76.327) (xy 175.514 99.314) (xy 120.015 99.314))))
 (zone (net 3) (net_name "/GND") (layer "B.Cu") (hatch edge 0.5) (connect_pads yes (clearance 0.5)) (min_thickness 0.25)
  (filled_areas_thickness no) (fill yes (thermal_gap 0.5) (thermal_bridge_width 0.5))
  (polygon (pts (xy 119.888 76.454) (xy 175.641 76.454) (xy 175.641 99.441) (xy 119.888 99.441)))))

